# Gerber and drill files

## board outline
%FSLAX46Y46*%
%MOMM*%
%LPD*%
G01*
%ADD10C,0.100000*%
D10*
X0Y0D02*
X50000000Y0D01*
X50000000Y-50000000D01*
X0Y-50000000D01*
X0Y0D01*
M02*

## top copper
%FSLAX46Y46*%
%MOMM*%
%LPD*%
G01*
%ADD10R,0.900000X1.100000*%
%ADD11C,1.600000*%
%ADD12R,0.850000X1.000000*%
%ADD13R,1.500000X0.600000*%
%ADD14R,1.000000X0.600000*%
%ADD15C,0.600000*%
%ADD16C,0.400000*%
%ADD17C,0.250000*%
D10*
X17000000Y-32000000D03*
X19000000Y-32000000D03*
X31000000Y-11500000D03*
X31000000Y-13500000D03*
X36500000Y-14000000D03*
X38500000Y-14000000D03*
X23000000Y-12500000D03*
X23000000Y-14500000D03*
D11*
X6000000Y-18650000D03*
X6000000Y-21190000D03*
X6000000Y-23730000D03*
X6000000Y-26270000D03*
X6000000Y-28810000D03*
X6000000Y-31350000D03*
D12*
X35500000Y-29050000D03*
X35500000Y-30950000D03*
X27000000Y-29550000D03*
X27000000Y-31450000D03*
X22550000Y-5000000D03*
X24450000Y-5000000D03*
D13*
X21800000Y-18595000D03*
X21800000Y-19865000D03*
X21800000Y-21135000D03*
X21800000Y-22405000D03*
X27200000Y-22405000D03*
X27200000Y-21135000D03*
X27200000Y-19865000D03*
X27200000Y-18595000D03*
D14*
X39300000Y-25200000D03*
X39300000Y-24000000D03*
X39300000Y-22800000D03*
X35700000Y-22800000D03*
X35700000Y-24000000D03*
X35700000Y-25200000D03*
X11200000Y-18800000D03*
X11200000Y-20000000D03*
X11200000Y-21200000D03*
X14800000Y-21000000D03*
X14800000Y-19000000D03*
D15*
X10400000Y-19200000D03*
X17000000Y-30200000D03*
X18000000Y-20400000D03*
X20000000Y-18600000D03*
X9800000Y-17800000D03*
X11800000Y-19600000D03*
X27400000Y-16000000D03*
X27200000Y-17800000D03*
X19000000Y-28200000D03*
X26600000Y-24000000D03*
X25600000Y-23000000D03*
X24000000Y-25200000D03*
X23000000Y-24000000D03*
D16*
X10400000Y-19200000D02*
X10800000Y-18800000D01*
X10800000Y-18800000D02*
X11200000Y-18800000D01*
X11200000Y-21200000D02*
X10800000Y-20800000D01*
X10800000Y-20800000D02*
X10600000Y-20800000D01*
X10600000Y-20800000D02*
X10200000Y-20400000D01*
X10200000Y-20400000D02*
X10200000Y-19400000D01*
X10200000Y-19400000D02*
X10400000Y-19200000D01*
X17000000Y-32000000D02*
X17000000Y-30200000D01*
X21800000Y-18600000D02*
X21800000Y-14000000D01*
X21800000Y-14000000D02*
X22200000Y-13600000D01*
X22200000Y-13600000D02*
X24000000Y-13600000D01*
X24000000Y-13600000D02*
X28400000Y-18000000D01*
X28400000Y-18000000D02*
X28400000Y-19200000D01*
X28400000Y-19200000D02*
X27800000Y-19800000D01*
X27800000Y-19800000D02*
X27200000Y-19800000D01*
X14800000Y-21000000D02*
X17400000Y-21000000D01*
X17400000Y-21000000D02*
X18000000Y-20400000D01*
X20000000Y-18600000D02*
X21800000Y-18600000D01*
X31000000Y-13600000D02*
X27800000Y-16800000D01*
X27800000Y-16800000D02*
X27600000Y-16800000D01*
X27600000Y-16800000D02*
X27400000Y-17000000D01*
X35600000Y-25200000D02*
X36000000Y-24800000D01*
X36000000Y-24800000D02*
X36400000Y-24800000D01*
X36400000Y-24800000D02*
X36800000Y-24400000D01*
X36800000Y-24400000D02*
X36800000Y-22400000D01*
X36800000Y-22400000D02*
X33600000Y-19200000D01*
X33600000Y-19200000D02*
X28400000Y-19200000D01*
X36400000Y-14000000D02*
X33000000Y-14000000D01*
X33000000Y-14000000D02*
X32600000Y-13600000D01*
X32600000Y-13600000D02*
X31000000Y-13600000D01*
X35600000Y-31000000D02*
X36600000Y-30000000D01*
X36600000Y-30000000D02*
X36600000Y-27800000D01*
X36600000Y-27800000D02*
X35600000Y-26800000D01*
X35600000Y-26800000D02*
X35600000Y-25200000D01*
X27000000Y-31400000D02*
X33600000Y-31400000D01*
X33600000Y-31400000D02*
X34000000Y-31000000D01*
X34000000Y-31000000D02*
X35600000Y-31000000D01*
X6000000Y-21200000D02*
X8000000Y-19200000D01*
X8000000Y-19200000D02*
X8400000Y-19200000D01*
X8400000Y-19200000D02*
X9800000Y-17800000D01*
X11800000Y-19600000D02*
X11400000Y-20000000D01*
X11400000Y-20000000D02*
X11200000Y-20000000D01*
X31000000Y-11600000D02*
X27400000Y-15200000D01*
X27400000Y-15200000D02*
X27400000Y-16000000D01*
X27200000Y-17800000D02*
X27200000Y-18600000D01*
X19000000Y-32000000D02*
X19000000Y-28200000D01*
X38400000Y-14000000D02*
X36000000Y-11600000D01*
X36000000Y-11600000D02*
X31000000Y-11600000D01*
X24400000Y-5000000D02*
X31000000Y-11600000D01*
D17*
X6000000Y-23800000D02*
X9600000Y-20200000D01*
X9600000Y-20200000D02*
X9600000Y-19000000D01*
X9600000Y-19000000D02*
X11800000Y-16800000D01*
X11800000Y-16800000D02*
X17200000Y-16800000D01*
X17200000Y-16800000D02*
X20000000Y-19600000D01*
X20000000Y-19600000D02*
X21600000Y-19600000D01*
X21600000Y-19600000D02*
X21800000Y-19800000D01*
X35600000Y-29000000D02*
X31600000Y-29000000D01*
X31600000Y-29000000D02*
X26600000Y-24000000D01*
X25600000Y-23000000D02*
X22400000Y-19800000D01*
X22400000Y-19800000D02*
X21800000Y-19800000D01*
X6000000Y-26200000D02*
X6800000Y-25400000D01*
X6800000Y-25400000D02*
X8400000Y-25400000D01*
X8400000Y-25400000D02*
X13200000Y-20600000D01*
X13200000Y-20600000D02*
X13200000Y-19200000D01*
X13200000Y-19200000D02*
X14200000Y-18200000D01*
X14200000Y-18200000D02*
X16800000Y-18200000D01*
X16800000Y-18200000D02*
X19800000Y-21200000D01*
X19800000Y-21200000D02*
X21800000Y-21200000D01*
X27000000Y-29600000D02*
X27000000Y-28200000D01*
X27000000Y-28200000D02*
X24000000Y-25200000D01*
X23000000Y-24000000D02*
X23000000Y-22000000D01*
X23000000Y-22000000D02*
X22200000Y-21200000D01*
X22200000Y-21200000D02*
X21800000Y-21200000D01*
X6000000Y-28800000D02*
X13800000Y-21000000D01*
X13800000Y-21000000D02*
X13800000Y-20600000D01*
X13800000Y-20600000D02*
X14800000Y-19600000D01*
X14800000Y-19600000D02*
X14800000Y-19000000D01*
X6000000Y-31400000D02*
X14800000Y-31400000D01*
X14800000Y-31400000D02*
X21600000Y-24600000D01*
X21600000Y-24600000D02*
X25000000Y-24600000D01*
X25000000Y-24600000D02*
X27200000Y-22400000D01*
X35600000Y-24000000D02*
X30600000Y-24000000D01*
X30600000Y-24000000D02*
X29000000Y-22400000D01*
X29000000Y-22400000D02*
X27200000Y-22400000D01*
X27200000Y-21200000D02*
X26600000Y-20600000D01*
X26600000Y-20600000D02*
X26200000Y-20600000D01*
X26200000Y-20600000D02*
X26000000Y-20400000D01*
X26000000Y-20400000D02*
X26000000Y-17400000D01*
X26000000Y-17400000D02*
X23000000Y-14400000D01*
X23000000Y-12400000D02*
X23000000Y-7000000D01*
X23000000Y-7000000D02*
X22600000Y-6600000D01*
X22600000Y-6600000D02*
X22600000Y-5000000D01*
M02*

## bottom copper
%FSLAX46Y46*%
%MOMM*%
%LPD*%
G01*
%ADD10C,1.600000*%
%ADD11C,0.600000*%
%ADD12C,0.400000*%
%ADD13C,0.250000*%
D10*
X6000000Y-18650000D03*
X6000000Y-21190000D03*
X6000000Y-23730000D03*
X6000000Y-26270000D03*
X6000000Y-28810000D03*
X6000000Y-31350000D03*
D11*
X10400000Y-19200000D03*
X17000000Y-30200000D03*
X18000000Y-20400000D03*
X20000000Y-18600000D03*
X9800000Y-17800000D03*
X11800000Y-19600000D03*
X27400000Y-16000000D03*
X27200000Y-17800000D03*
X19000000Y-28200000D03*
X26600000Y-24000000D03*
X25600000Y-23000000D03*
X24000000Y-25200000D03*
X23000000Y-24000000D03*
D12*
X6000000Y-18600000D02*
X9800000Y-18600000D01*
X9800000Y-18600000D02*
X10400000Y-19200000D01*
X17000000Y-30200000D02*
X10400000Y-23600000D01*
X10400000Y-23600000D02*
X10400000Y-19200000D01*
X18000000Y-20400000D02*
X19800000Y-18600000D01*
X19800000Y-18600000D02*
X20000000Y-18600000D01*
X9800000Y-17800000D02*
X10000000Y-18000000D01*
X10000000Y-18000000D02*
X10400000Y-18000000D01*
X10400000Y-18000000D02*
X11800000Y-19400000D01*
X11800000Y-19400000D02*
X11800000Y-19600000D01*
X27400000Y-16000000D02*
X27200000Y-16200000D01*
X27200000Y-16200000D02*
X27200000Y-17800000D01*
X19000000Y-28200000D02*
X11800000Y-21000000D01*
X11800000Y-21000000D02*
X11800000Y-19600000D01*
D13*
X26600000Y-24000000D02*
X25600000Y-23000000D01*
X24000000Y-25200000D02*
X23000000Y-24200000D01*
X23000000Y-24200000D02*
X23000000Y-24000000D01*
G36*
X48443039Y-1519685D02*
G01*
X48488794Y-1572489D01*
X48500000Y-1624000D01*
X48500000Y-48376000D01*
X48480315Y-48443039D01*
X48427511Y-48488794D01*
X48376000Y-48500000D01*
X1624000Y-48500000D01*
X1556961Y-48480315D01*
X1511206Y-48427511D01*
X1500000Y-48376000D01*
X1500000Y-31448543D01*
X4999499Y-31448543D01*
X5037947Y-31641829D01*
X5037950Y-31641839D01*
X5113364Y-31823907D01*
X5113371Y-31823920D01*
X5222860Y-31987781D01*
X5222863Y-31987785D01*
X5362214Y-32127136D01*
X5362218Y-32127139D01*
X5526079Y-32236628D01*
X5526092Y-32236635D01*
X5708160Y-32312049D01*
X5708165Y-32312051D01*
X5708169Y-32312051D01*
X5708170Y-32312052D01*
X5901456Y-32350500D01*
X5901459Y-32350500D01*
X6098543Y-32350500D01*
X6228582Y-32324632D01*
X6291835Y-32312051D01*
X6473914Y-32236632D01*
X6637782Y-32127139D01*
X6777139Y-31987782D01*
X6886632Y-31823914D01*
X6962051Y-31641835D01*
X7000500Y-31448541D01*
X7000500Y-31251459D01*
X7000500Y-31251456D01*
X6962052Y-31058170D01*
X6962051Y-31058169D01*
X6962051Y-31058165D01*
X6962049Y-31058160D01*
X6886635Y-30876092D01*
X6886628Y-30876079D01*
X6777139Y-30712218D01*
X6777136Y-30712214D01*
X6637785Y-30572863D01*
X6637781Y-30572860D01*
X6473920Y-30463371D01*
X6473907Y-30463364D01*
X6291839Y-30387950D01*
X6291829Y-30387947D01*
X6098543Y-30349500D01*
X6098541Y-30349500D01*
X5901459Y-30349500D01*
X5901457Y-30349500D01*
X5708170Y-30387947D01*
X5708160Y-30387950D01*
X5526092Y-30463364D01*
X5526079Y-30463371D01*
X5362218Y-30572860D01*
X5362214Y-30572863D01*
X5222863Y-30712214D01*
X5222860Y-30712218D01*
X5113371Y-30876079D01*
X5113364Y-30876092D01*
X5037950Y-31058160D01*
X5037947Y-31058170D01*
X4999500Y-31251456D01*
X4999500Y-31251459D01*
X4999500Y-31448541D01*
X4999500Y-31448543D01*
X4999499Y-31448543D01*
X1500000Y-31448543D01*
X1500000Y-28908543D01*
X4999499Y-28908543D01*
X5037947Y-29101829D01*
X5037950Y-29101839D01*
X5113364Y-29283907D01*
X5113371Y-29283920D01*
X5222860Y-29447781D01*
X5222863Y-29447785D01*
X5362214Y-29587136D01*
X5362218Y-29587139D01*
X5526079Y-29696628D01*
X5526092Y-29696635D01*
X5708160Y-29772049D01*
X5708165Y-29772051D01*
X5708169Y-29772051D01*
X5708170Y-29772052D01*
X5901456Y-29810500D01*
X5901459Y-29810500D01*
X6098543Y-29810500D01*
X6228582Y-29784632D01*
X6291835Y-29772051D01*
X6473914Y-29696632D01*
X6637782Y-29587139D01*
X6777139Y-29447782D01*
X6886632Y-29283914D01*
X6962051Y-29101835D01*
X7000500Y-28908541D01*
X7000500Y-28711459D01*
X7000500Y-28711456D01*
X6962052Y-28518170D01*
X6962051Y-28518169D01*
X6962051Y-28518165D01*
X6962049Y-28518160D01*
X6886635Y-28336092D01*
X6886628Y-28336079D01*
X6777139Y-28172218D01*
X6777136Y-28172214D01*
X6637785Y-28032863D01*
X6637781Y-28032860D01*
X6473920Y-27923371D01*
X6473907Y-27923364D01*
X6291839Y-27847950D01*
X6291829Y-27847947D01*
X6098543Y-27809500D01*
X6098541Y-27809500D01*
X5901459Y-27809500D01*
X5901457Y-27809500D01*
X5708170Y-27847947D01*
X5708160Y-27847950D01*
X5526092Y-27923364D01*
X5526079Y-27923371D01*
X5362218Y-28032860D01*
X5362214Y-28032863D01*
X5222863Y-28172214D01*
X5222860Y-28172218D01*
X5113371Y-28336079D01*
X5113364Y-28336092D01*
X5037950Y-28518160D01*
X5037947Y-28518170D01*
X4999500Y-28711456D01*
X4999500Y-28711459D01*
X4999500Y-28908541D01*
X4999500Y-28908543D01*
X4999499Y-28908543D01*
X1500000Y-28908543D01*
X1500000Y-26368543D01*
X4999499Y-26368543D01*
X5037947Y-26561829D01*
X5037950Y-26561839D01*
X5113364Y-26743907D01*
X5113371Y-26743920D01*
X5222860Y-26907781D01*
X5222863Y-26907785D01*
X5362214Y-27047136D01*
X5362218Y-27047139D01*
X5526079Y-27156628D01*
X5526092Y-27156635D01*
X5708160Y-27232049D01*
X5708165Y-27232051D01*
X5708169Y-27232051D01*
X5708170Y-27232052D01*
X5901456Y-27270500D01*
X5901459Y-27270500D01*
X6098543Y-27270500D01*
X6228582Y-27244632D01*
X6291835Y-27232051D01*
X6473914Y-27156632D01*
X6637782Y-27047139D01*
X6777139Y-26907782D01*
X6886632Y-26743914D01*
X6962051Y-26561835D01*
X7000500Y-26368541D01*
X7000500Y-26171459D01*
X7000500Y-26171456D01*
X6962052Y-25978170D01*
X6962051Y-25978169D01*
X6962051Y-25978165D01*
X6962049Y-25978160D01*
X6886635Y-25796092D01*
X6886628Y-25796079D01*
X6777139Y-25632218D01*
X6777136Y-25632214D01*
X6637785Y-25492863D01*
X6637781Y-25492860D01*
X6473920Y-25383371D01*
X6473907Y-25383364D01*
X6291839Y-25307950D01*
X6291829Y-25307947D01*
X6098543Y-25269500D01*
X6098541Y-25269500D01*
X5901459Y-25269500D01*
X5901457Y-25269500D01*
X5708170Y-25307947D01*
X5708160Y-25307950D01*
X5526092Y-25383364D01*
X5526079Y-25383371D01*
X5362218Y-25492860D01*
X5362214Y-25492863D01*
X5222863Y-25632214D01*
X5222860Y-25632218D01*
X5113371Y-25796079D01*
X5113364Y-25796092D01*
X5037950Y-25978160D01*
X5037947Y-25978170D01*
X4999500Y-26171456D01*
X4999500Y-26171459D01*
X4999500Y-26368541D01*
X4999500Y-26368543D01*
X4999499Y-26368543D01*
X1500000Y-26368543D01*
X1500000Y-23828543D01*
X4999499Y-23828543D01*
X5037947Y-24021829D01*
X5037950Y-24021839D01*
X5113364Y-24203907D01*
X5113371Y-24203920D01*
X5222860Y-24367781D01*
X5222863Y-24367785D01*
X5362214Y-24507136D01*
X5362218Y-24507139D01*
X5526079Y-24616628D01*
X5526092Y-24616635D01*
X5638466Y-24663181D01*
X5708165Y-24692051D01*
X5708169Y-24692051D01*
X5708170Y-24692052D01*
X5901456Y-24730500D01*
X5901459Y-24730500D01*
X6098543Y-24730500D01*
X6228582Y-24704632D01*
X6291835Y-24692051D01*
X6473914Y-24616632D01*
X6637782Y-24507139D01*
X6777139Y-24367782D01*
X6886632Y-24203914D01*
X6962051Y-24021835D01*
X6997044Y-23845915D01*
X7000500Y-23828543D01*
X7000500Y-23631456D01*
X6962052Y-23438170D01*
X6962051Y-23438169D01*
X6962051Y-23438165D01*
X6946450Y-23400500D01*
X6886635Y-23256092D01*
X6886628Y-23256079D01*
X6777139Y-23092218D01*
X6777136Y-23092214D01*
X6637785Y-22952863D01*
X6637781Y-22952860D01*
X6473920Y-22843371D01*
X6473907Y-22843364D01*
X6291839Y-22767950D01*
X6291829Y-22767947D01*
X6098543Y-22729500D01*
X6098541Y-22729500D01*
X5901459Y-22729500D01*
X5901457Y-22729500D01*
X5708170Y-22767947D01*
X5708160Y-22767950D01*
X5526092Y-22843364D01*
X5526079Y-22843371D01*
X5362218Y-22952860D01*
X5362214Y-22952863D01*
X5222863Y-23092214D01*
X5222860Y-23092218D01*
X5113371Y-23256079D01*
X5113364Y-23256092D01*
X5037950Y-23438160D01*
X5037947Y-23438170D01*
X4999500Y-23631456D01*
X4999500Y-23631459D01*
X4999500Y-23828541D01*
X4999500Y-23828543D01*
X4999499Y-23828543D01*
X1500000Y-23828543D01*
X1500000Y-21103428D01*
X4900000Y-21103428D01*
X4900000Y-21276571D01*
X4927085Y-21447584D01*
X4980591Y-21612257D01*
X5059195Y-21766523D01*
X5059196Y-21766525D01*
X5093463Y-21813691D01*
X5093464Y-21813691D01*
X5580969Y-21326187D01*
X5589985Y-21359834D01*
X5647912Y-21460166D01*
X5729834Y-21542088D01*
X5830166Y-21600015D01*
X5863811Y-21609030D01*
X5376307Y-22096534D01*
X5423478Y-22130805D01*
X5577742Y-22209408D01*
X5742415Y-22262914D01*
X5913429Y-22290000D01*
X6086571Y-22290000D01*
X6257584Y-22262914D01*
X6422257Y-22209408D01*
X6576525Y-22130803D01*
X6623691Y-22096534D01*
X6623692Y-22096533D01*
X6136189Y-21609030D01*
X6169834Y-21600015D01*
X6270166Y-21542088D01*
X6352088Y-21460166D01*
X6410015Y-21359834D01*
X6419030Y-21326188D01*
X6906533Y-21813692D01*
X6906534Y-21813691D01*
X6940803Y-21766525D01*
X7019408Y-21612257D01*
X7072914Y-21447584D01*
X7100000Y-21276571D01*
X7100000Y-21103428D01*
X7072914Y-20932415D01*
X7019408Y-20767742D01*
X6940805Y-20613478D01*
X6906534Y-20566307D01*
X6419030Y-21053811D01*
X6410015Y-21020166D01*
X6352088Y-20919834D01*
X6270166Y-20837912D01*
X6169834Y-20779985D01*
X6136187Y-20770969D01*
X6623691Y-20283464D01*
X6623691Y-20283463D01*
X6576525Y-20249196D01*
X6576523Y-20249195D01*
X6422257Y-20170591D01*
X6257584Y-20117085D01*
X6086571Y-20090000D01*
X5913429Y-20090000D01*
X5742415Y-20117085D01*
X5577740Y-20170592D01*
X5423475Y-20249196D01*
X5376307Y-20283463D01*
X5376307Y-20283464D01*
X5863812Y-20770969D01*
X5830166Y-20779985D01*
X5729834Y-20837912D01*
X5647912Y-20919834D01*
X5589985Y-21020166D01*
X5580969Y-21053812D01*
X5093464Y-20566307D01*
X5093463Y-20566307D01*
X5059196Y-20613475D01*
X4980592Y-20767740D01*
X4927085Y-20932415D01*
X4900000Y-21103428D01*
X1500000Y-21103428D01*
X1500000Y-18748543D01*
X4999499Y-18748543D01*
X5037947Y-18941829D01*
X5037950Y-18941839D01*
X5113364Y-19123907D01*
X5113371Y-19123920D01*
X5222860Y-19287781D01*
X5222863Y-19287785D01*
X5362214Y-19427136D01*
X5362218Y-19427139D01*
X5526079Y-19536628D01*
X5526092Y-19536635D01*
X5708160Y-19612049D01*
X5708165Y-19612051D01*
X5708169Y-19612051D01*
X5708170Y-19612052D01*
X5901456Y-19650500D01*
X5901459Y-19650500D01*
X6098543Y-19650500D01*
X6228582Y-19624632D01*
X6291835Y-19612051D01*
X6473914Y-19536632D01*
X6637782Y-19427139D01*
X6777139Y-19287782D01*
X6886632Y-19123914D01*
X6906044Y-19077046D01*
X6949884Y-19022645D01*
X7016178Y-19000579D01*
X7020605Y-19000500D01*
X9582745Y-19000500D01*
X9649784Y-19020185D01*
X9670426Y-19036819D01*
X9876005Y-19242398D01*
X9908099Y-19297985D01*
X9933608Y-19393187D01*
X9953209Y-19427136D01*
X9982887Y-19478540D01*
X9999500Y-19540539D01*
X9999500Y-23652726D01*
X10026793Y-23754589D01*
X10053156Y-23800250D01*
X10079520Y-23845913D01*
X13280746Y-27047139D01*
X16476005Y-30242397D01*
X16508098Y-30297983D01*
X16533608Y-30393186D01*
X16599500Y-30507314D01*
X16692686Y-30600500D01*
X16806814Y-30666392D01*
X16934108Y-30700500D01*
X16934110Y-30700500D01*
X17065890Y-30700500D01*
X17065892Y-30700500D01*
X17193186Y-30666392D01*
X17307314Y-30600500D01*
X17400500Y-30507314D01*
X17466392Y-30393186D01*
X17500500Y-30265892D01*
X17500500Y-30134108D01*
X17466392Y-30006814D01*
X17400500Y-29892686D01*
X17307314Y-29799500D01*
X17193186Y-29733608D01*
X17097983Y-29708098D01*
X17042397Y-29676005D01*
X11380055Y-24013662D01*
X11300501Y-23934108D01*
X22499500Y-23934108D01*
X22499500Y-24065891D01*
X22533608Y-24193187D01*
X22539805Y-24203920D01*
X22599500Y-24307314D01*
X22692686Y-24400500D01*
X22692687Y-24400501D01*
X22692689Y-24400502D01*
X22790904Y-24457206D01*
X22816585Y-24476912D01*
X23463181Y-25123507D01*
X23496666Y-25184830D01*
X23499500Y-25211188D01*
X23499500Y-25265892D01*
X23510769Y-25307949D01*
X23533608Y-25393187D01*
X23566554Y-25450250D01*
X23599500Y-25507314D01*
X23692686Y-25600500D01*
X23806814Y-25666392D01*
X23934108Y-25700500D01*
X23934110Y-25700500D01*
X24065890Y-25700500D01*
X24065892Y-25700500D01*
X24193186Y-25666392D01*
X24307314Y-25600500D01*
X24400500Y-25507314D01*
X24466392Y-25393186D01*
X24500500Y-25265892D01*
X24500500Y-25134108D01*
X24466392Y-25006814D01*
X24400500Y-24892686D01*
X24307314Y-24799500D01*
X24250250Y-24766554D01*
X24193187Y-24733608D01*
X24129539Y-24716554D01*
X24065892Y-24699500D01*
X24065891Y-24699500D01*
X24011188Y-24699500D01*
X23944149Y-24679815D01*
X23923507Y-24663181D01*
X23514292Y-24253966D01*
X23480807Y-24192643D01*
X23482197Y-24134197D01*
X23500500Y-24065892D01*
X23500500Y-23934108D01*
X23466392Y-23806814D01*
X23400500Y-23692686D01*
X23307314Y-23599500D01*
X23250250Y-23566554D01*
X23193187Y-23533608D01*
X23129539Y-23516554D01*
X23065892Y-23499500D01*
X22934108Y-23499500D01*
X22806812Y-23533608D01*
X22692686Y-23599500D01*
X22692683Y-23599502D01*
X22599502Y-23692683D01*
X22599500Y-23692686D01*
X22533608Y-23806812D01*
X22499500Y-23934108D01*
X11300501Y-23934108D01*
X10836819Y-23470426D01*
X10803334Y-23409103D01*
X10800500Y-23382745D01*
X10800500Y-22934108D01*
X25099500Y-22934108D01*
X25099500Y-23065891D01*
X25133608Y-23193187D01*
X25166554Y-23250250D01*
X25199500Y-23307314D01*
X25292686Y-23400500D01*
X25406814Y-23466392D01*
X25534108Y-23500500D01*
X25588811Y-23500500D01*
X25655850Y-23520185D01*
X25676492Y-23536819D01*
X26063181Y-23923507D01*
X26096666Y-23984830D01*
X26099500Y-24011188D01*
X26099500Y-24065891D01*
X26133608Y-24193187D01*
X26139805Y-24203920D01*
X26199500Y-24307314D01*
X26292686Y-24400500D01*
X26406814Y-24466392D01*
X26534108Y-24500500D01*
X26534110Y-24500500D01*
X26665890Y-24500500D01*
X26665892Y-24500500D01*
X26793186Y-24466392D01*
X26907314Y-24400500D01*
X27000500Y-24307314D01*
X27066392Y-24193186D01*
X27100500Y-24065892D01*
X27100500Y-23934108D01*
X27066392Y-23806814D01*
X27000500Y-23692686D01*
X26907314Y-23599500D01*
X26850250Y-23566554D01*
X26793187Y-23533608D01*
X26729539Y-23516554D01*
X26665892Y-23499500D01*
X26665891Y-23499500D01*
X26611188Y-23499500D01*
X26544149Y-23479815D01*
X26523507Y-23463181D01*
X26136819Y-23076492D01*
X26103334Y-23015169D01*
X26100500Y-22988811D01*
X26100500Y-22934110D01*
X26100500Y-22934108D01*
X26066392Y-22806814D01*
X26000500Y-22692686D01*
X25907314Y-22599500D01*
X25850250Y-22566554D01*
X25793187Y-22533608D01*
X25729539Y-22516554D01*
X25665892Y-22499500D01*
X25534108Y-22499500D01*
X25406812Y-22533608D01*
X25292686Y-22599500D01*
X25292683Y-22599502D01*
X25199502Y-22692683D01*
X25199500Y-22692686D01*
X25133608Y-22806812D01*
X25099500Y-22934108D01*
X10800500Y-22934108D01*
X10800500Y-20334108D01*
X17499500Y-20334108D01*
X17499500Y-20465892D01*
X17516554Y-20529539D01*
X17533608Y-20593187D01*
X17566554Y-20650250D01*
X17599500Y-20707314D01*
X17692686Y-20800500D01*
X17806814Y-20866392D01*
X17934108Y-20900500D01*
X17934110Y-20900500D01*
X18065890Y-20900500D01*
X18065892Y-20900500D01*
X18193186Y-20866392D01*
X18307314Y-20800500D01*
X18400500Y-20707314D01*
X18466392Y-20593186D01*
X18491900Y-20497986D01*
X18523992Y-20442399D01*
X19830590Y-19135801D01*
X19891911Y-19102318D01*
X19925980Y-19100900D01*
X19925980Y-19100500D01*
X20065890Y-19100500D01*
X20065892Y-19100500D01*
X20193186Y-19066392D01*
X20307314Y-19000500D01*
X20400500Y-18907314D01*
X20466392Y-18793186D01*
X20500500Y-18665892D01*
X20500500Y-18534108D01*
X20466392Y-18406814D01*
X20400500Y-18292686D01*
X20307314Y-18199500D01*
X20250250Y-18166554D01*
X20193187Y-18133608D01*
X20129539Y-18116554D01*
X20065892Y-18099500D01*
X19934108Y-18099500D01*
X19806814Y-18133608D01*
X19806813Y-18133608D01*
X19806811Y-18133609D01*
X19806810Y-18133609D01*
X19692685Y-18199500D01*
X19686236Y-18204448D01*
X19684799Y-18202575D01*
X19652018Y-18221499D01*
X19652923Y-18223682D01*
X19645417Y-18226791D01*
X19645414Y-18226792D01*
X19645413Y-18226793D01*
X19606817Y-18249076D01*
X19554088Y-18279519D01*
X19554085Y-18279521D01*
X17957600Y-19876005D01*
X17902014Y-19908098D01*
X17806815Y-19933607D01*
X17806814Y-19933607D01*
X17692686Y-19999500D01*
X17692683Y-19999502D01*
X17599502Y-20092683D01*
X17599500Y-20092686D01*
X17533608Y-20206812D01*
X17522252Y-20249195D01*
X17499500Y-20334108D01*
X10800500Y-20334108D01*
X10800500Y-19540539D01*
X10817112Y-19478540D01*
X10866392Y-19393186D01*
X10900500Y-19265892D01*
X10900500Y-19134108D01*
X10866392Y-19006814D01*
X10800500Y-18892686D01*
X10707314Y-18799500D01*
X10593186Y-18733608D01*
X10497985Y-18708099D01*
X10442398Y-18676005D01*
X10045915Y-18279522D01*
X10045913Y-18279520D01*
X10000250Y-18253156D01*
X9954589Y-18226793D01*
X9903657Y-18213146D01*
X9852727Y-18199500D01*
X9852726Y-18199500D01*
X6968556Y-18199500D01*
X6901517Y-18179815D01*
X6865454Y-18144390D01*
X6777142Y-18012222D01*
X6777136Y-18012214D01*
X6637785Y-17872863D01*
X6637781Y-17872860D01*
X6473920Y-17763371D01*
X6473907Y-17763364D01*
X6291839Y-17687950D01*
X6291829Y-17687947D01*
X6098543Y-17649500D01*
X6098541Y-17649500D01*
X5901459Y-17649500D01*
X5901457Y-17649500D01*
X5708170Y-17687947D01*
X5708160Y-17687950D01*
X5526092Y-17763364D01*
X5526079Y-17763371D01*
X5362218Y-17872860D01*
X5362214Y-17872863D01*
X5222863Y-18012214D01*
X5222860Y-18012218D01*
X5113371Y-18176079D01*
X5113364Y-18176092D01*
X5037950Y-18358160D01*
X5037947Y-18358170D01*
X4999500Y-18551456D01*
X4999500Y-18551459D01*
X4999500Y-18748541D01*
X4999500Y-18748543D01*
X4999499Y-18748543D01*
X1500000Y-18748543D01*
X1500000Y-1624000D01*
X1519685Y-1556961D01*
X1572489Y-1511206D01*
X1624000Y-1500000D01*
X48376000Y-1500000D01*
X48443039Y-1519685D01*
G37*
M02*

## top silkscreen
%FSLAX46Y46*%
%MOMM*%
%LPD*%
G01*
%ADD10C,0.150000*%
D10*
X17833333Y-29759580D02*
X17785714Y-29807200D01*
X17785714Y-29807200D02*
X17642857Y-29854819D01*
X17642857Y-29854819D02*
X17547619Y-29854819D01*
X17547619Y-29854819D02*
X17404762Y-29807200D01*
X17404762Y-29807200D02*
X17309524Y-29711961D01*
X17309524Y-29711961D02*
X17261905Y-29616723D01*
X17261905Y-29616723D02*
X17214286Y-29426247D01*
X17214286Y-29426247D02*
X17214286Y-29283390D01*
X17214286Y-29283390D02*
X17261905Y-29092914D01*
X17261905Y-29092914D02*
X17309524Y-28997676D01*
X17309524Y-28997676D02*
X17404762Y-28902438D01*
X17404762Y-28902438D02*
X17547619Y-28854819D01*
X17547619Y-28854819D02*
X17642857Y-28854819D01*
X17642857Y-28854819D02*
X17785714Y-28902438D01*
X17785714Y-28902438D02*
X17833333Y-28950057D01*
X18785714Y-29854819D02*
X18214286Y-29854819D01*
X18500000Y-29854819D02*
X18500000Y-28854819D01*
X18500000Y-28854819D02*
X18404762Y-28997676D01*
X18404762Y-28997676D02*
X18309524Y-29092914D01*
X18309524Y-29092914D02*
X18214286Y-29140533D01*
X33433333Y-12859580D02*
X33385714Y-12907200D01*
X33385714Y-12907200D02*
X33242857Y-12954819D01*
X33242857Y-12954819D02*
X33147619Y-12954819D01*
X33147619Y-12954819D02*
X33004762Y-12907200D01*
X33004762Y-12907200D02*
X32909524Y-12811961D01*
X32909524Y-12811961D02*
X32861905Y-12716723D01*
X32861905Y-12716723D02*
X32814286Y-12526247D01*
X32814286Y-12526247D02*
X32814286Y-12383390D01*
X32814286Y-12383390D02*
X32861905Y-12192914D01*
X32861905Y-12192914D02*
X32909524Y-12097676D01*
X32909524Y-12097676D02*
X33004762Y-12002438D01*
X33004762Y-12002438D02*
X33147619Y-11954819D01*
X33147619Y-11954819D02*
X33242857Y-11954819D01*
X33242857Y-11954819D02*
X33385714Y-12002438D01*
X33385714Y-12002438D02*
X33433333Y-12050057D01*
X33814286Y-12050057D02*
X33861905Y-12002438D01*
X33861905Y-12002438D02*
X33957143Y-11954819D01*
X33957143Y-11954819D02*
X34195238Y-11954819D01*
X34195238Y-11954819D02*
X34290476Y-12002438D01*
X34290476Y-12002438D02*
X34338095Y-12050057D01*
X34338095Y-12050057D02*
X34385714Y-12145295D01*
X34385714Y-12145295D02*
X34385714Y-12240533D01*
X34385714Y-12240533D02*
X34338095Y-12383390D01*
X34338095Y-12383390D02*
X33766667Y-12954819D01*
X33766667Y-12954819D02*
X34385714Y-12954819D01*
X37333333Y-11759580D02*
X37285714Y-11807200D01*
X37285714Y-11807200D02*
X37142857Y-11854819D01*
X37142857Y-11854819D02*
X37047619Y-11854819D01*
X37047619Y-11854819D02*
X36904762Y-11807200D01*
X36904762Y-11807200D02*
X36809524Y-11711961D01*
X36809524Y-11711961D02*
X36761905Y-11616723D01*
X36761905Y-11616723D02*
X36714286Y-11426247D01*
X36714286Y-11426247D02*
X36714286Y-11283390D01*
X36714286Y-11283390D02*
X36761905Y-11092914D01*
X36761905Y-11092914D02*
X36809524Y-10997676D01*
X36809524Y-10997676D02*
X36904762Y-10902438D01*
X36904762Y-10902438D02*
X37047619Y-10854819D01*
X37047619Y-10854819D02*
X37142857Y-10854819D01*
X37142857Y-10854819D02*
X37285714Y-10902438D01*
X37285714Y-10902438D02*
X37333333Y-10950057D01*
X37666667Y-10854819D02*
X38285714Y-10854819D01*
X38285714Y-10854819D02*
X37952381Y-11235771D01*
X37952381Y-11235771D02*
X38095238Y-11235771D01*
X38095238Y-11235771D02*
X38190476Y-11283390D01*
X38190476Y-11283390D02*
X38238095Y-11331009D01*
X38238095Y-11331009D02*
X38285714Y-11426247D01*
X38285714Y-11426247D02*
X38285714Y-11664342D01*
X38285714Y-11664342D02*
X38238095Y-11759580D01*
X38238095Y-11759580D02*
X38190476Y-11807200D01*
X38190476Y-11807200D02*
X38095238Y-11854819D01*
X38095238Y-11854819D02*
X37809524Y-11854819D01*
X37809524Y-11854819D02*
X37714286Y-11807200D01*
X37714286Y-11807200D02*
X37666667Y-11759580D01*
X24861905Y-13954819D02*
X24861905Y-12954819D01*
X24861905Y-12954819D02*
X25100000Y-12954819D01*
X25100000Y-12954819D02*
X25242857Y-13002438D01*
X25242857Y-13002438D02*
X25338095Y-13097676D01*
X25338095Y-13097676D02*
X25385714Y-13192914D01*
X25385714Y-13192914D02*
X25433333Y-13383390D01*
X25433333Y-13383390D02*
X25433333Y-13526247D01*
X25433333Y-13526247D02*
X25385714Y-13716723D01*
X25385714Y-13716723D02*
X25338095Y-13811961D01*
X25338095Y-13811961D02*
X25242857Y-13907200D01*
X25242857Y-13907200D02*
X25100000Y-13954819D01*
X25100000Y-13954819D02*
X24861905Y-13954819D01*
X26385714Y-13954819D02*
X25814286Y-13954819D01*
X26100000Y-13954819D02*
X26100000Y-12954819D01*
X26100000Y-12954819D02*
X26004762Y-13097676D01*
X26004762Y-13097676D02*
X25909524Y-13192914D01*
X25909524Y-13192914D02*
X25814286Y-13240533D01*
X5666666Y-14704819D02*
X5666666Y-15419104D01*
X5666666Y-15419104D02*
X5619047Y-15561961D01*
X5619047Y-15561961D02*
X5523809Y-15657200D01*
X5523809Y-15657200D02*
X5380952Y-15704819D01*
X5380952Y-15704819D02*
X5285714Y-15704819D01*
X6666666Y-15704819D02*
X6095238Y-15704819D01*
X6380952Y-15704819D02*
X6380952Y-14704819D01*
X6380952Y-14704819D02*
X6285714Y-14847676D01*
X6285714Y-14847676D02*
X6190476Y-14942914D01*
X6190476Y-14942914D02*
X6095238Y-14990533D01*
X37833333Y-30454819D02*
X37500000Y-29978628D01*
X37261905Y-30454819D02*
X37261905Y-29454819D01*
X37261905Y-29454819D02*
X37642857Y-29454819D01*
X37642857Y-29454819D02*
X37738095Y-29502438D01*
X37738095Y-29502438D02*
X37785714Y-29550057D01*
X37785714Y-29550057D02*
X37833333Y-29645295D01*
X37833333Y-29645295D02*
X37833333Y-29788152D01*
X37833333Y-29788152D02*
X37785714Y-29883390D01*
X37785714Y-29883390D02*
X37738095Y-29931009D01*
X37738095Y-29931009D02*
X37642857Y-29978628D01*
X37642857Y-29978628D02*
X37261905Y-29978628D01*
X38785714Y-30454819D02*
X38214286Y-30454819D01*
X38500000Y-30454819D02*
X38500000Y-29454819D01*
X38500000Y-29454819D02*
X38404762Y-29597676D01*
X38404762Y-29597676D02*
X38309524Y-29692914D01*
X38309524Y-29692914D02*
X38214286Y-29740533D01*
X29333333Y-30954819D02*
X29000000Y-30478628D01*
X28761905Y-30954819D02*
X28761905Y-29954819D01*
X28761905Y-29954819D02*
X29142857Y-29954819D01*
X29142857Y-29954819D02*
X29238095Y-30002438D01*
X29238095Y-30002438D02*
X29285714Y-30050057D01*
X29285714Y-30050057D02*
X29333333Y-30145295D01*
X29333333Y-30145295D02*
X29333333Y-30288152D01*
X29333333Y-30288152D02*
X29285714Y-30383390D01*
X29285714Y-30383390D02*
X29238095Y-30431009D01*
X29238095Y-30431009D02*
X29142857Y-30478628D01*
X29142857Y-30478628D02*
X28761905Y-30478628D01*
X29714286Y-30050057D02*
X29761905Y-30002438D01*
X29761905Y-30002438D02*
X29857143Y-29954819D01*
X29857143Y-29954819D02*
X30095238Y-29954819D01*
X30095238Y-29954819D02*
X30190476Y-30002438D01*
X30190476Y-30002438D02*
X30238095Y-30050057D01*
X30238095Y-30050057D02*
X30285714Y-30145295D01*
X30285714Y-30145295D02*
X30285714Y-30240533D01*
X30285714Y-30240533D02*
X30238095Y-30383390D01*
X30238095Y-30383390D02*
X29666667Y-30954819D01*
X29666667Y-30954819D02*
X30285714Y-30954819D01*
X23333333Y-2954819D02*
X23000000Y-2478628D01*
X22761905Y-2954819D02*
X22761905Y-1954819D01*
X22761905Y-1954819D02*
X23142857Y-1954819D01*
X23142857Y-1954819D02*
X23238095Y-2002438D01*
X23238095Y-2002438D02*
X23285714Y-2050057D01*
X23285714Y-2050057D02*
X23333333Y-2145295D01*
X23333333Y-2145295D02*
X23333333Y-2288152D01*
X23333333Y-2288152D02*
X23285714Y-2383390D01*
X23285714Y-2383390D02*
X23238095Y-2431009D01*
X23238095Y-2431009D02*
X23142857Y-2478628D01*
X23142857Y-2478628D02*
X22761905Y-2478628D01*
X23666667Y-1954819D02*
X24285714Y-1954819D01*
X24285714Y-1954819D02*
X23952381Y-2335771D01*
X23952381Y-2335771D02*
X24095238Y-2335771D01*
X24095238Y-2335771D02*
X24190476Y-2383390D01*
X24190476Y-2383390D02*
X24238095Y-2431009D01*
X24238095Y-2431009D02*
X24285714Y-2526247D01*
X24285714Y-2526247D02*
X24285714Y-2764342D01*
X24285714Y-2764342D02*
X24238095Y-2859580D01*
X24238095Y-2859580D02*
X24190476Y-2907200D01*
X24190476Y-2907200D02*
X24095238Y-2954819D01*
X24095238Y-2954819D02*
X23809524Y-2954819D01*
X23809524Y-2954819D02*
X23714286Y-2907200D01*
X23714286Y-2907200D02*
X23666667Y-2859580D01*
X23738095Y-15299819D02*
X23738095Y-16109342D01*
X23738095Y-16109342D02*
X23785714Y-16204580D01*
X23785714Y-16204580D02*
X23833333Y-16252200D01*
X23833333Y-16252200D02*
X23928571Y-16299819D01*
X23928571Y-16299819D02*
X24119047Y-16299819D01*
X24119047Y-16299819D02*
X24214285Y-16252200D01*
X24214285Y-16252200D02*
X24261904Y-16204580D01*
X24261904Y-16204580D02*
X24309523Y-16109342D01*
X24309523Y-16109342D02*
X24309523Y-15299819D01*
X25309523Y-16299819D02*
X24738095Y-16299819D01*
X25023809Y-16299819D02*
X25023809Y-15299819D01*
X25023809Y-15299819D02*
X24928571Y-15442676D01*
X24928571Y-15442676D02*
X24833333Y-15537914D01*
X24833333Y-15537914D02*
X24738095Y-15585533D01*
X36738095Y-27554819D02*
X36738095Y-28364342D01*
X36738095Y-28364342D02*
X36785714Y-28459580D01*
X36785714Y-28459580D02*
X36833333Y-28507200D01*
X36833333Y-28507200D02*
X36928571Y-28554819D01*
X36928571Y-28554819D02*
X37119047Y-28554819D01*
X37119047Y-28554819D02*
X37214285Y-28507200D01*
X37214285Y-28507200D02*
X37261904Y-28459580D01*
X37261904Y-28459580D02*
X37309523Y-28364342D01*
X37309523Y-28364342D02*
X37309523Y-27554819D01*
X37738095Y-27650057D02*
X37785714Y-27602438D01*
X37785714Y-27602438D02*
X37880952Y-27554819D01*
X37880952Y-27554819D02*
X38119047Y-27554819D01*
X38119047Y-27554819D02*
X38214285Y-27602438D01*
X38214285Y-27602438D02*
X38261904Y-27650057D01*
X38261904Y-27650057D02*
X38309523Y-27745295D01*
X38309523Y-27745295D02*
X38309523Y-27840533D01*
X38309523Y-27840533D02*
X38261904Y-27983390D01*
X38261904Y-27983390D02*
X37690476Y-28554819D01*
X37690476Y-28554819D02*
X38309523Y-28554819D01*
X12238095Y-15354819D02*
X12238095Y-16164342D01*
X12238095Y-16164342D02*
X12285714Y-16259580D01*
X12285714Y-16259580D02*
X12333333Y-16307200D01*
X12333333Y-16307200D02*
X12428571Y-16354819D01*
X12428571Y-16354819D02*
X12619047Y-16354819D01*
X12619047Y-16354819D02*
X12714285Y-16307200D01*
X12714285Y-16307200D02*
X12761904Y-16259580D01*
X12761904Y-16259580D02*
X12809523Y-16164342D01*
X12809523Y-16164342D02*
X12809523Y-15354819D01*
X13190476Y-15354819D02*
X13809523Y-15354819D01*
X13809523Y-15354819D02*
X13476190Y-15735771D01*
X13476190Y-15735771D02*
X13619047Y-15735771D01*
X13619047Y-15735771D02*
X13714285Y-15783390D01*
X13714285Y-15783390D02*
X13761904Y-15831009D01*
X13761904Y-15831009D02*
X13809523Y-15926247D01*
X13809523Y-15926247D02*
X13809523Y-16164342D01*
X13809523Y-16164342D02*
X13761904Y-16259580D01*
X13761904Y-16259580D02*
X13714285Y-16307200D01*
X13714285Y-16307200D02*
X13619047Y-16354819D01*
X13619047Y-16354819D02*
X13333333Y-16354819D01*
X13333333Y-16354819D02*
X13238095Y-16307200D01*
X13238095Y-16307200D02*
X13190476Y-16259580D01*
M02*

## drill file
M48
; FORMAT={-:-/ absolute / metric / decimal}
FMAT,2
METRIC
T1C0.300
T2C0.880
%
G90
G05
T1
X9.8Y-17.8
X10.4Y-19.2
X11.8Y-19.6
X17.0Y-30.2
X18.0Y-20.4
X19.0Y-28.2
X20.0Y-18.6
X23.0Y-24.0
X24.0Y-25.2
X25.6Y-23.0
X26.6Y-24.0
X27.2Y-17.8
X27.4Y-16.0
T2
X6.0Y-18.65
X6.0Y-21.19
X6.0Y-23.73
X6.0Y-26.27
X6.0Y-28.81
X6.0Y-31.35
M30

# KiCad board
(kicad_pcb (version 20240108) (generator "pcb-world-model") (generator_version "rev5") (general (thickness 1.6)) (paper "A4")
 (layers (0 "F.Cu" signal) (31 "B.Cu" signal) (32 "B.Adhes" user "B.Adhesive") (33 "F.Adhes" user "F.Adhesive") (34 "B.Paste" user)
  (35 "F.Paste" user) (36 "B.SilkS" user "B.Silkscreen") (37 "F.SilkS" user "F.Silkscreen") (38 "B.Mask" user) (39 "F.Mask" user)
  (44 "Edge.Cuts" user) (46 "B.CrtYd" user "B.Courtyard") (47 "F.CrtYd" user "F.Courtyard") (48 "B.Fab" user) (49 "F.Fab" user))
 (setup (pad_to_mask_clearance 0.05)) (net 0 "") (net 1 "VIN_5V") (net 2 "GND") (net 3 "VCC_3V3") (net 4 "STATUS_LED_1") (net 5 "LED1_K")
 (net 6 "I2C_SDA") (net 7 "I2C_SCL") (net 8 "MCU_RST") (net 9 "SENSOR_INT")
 (gr_rect (start 0.0 0.0) (end 50.0000 50.0000) (stroke (width 0.1) (type default)) (fill none) (layer "Edge.Cuts"))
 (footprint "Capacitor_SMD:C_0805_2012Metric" (layer "F.Cu") (at 18.0000 32.0000 0)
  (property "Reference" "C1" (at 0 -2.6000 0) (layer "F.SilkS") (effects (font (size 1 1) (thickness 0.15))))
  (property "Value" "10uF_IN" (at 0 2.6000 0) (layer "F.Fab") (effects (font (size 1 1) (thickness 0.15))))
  (pad "1" smd rect (at -1.0000 0.0000) (size 0.9000 1.1000) (layers "F.Cu" "F.Paste" "F.Mask") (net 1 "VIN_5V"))
  (pad "2" smd rect (at 1.0000 0.0000) (size 0.9000 1.1000) (layers "F.Cu" "F.Paste" "F.Mask") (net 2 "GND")))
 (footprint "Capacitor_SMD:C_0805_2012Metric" (layer "F.Cu") (at 31.0000 12.5000 270)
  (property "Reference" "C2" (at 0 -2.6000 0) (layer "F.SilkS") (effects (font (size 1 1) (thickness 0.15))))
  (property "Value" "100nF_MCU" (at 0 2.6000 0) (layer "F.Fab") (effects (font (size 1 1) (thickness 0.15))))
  (pad "1" smd rect (at -1.0000 0.0000) (size 0.9000 1.1000) (layers "F.Cu" "F.Paste" "F.Mask") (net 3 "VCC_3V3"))
  (pad "2" smd rect (at 1.0000 0.0000) (size 0.9000 1.1000) (layers "F.Cu" "F.Paste" "F.Mask") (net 2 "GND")))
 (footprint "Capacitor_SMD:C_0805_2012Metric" (layer "F.Cu") (at 37.5000 14.0000 0)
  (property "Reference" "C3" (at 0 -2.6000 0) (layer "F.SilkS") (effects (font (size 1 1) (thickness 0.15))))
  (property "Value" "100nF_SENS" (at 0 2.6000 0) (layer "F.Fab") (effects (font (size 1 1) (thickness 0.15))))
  (pad "1" smd rect (at -1.0000 0.0000) (size 0.9000 1.1000) (layers "F.Cu" "F.Paste" "F.Mask") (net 3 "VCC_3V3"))
  (pad "2" smd rect (at 1.0000 0.0000) (size 0.9000 1.1000) (layers "F.Cu" "F.Paste" "F.Mask") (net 2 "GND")))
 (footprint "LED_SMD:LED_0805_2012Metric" (layer "F.Cu") (at 23.0000 13.5000 270)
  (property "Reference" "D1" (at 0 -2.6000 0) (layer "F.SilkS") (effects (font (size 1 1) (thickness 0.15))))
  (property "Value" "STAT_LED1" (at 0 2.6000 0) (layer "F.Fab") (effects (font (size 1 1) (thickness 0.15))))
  (pad "1" smd rect (at -1.0000 0.0000) (size 0.9000 1.1000) (layers "F.Cu" "F.Paste" "F.Mask") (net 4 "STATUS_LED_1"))
  (pad "2" smd rect (at 1.0000 0.0000) (size 0.9000 1.1000) (layers "F.Cu" "F.Paste" "F.Mask") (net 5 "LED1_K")))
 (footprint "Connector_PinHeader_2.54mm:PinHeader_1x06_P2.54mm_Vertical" (layer "F.Cu") (at 6.0000 25.0000 0) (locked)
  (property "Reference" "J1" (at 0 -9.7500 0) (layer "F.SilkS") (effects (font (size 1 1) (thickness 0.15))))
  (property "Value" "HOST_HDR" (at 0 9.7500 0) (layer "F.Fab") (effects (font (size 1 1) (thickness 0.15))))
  (pad "1" thru_hole circle (at 0.0000 -6.3500) (size 1.6000 1.6000) (drill 0.8800) (layers "*.Cu" "*.Mask") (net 1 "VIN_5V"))
  (pad "2" thru_hole circle (at 0.0000 -3.8100) (size 1.6000 1.6000) (drill 0.8800) (layers "*.Cu" "*.Mask") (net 2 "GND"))
  (pad "3" thru_hole circle (at 0.0000 -1.2700) (size 1.6000 1.6000) (drill 0.8800) (layers "*.Cu" "*.Mask") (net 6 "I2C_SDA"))
  (pad "4" thru_hole circle (at 0.0000 1.2700) (size 1.6000 1.6000) (drill 0.8800) (layers "*.Cu" "*.Mask") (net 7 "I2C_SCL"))
  (pad "5" thru_hole circle (at 0.0000 3.8100) (size 1.6000 1.6000) (drill 0.8800) (layers "*.Cu" "*.Mask") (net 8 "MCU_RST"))
  (pad "6" thru_hole circle (at 0.0000 6.3500) (size 1.6000 1.6000) (drill 0.8800) (layers "*.Cu" "*.Mask") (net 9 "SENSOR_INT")))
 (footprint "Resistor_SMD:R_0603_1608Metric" (layer "F.Cu") (at 35.5000 30.0000 270)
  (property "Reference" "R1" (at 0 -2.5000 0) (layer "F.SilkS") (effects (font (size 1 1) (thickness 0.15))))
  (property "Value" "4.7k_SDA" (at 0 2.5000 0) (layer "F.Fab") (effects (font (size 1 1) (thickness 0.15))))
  (pad "1" smd rect (at -0.9500 0.0000) (size 0.8500 1.0000) (layers "F.Cu" "F.Paste" "F.Mask") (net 3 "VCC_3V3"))
  (pad "2" smd rect (at 0.9500 0.0000) (size 0.8500 1.0000) (layers "F.Cu" "F.Paste" "F.Mask") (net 6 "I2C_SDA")))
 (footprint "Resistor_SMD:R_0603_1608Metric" (layer "F.Cu") (at 27.0000 30.5000 270)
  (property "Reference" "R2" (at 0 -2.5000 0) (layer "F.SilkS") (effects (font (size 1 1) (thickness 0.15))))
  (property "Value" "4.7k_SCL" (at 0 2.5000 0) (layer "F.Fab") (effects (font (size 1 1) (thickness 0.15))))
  (pad "1" smd rect (at -0.9500 0.0000) (size 0.8500 1.0000) (layers "F.Cu" "F.Paste" "F.Mask") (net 3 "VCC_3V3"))
  (pad "2" smd rect (at 0.9500 0.0000) (size 0.8500 1.0000) (layers "F.Cu" "F.Paste" "F.Mask") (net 7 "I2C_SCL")))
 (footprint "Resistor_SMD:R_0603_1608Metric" (layer "F.Cu") (at 23.5000 5.0000 0)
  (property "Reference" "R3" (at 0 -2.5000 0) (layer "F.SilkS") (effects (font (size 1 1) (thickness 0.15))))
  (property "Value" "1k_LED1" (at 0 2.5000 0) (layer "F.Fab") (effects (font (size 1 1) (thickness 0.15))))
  (pad "1" smd rect (at -0.9500 0.0000) (size 0.8500 1.0000) (layers "F.Cu" "F.Paste" "F.Mask") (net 5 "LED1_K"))
  (pad "2" smd rect (at 0.9500 0.0000) (size 0.8500 1.0000) (layers "F.Cu" "F.Paste" "F.Mask") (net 2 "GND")))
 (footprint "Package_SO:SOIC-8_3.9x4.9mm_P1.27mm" (layer "F.Cu") (at 24.5000 20.5000 0)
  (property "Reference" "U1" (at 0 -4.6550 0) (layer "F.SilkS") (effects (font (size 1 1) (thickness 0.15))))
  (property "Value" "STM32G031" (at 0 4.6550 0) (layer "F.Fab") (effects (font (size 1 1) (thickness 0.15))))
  (pad "1" smd rect (at -2.7000 -1.9050) (size 1.5000 0.6000) (layers "F.Cu" "F.Paste" "F.Mask") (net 3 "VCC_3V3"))
  (pad "2" smd rect (at -2.7000 -0.6350) (size 1.5000 0.6000) (layers "F.Cu" "F.Paste" "F.Mask") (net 6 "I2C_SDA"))
  (pad "3" smd rect (at -2.7000 0.6350) (size 1.5000 0.6000) (layers "F.Cu" "F.Paste" "F.Mask") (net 7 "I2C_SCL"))
  (pad "4" smd rect (at -2.7000 1.9050) (size 1.5000 0.6000) (layers "F.Cu" "F.Paste" "F.Mask") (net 8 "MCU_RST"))
  (pad "5" smd rect (at 2.7000 1.9050) (size 1.5000 0.6000) (layers "F.Cu" "F.Paste" "F.Mask") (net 9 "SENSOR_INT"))
  (pad "6" smd rect (at 2.7000 0.6350) (size 1.5000 0.6000) (layers "F.Cu" "F.Paste" "F.Mask") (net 4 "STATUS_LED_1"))
  (pad "7" smd rect (at 2.7000 -0.6350) (size 1.5000 0.6000) (layers "F.Cu" "F.Paste" "F.Mask") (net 3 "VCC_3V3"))
  (pad "8" smd rect (at 2.7000 -1.9050) (size 1.5000 0.6000) (layers "F.Cu" "F.Paste" "F.Mask") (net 2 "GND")))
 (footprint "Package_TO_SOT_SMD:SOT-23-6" (layer "F.Cu") (at 37.5000 24.0000 180)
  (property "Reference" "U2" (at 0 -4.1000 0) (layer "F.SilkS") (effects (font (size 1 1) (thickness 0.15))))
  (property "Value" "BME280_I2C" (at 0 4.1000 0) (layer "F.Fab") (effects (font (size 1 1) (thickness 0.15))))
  (pad "1" smd rect (at -1.8000 -1.2000) (size 1.0000 0.6000) (layers "F.Cu" "F.Paste" "F.Mask") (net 3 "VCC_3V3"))
  (pad "2" smd rect (at -1.8000 0.0000) (size 1.0000 0.6000) (layers "F.Cu" "F.Paste" "F.Mask") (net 2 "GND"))
  (pad "3" smd rect (at -1.8000 1.2000) (size 1.0000 0.6000) (layers "F.Cu" "F.Paste" "F.Mask") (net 6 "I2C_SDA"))
  (pad "4" smd rect (at 1.8000 1.2000) (size 1.0000 0.6000) (layers "F.Cu" "F.Paste" "F.Mask") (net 7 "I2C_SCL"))
  (pad "5" smd rect (at 1.8000 0.0000) (size 1.0000 0.6000) (layers "F.Cu" "F.Paste" "F.Mask") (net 9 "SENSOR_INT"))
  (pad "6" smd rect (at 1.8000 -1.2000) (size 1.0000 0.6000) (layers "F.Cu" "F.Paste" "F.Mask") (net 3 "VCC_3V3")))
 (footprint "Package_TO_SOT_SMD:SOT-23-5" (layer "F.Cu") (at 13.0000 20.0000 0)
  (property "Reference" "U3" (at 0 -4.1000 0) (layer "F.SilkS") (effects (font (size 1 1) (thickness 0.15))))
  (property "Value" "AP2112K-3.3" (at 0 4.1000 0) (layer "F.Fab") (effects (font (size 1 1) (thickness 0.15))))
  (pad "1" smd rect (at -1.8000 -1.2000) (size 1.0000 0.6000) (layers "F.Cu" "F.Paste" "F.Mask") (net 1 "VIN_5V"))
  (pad "2" smd rect (at -1.8000 0.0000) (size 1.0000 0.6000) (layers "F.Cu" "F.Paste" "F.Mask") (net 2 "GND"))
  (pad "3" smd rect (at -1.8000 1.2000) (size 1.0000 0.6000) (layers "F.Cu" "F.Paste" "F.Mask") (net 1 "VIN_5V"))
  (pad "4" smd rect (at 1.8000 1.0000) (size 1.0000 0.6000) (layers "F.Cu" "F.Paste" "F.Mask") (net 3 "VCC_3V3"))
  (pad "5" smd rect (at 1.8000 -1.0000) (size 1.0000 0.6000) (layers "F.Cu" "F.Paste" "F.Mask") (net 8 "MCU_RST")))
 (segment (start 6.0000 18.6000) (end 9.8000 18.6000) (width 0.4000) (layer "B.Cu") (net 1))
 (segment (start 9.8000 18.6000) (end 10.4000 19.2000) (width 0.4000) (layer "B.Cu") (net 1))
 (segment (start 10.4000 19.2000) (end 10.8000 18.8000) (width 0.4000) (layer "F.Cu") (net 1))
 (segment (start 10.8000 18.8000) (end 11.2000 18.8000) (width 0.4000) (layer "F.Cu") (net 1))
 (segment (start 11.2000 21.2000) (end 10.8000 20.8000) (width 0.4000) (layer "F.Cu") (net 1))
 (segment (start 10.8000 20.8000) (end 10.6000 20.8000) (width 0.4000) (layer "F.Cu") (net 1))
 (segment (start 10.6000 20.8000) (end 10.2000 20.4000) (width 0.4000) (layer "F.Cu") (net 1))
 (segment (start 10.2000 20.4000) (end 10.2000 19.4000) (width 0.4000) (layer "F.Cu") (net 1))
 (segment (start 10.2000 19.4000) (end 10.4000 19.2000) (width 0.4000) (layer "F.Cu") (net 1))
 (segment (start 17.0000 32.0000) (end 17.0000 30.2000) (width 0.4000) (layer "F.Cu") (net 1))
 (segment (start 17.0000 30.2000) (end 10.4000 23.6000) (width 0.4000) (layer "B.Cu") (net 1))
 (segment (start 10.4000 23.6000) (end 10.4000 19.2000) (width 0.4000) (layer "B.Cu") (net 1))
 (segment (start 21.8000 18.6000) (end 21.8000 14.0000) (width 0.4000) (layer "F.Cu") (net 3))
 (segment (start 21.8000 14.0000) (end 22.2000 13.6000) (width 0.4000) (layer "F.Cu") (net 3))
 (segment (start 22.2000 13.6000) (end 24.0000 13.6000) (width 0.4000) (layer "F.Cu") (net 3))
 (segment (start 24.0000 13.6000) (end 28.4000 18.0000) (width 0.4000) (layer "F.Cu") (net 3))
 (segment (start 28.4000 18.0000) (end 28.4000 19.2000) (width 0.4000) (layer "F.Cu") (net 3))
 (segment (start 28.4000 19.2000) (end 27.8000 19.8000) (width 0.4000) (layer "F.Cu") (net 3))
 (segment (start 27.8000 19.8000) (end 27.2000 19.8000) (width 0.4000) (layer "F.Cu") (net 3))
 (segment (start 14.8000 21.0000) (end 17.4000 21.0000) (width 0.4000) (layer "F.Cu") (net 3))
 (segment (start 17.4000 21.0000) (end 18.0000 20.4000) (width 0.4000) (layer "F.Cu") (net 3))
 (segment (start 18.0000 20.4000) (end 19.8000 18.6000) (width 0.4000) (layer "B.Cu") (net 3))
 (segment (start 19.8000 18.6000) (end 20.0000 18.6000) (width 0.4000) (layer "B.Cu") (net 3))
 (segment (start 20.0000 18.6000) (end 21.8000 18.6000) (width 0.4000) (layer "F.Cu") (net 3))
 (segment (start 31.0000 13.6000) (end 27.8000 16.8000) (width 0.4000) (layer "F.Cu") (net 3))
 (segment (start 27.8000 16.8000) (end 27.6000 16.8000) (width 0.4000) (layer "F.Cu") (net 3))
 (segment (start 27.6000 16.8000) (end 27.4000 17.0000) (width 0.4000) (layer "F.Cu") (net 3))
 (segment (start 35.6000 25.2000) (end 36.0000 24.8000) (width 0.4000) (layer "F.Cu") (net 3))
 (segment (start 36.0000 24.8000) (end 36.4000 24.8000) (width 0.4000) (layer "F.Cu") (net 3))
 (segment (start 36.4000 24.8000) (end 36.8000 24.4000) (width 0.4000) (layer "F.Cu") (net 3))
 (segment (start 36.8000 24.4000) (end 36.8000 22.4000) (width 0.4000) (layer "F.Cu") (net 3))
 (segment (start 36.8000 22.4000) (end 33.6000 19.2000) (width 0.4000) (layer "F.Cu") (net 3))
 (segment (start 33.6000 19.2000) (end 28.4000 19.2000) (width 0.4000) (layer "F.Cu") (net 3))
 (segment (start 36.4000 14.0000) (end 33.0000 14.0000) (width 0.4000) (layer "F.Cu") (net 3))
 (segment (start 33.0000 14.0000) (end 32.6000 13.6000) (width 0.4000) (layer "F.Cu") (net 3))
 (segment (start 32.6000 13.6000) (end 31.0000 13.6000) (width 0.4000) (layer "F.Cu") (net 3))
 (segment (start 35.6000 31.0000) (end 36.6000 30.0000) (width 0.4000) (layer "F.Cu") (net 3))
 (segment (start 36.6000 30.0000) (end 36.6000 27.8000) (width 0.4000) (layer "F.Cu") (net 3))
 (segment (start 36.6000 27.8000) (end 35.6000 26.8000) (width 0.4000) (layer "F.Cu") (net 3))
 (segment (start 35.6000 26.8000) (end 35.6000 25.2000) (width 0.4000) (layer "F.Cu") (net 3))
 (segment (start 27.0000 31.4000) (end 33.6000 31.4000) (width 0.4000) (layer "F.Cu") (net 3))
 (segment (start 33.6000 31.4000) (end 34.0000 31.0000) (width 0.4000) (layer "F.Cu") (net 3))
 (segment (start 34.0000 31.0000) (end 35.6000 31.0000) (width 0.4000) (layer "F.Cu") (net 3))
 (segment (start 6.0000 21.2000) (end 8.0000 19.2000) (width 0.4000) (layer "F.Cu") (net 2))
 (segment (start 8.0000 19.2000) (end 8.4000 19.2000) (width 0.4000) (layer "F.Cu") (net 2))
 (segment (start 8.4000 19.2000) (end 9.8000 17.8000) (width 0.4000) (layer "F.Cu") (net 2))
 (segment (start 9.8000 17.8000) (end 10.0000 18.0000) (width 0.4000) (layer "B.Cu") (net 2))
 (segment (start 10.0000 18.0000) (end 10.4000 18.0000) (width 0.4000) (layer "B.Cu") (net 2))
 (segment (start 10.4000 18.0000) (end 11.8000 19.4000) (width 0.4000) (layer "B.Cu") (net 2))
 (segment (start 11.8000 19.4000) (end 11.8000 19.6000) (width 0.4000) (layer "B.Cu") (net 2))
 (segment (start 11.8000 19.6000) (end 11.4000 20.0000) (width 0.4000) (layer "F.Cu") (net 2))
 (segment (start 11.4000 20.0000) (end 11.2000 20.0000) (width 0.4000) (layer "F.Cu") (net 2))
 (segment (start 31.0000 11.6000) (end 27.4000 15.2000) (width 0.4000) (layer "F.Cu") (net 2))
 (segment (start 27.4000 15.2000) (end 27.4000 16.0000) (width 0.4000) (layer "F.Cu") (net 2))
 (segment (start 27.4000 16.0000) (end 27.2000 16.2000) (width 0.4000) (layer "B.Cu") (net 2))
 (segment (start 27.2000 16.2000) (end 27.2000 17.8000) (width 0.4000) (layer "B.Cu") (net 2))
 (segment (start 27.2000 17.8000) (end 27.2000 18.6000) (width 0.4000) (layer "F.Cu") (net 2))
 (segment (start 19.0000 32.0000) (end 19.0000 28.2000) (width 0.4000) (layer "F.Cu") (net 2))
 (segment (start 19.0000 28.2000) (end 11.8000 21.0000) (width 0.4000) (layer "B.Cu") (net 2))
 (segment (start 11.8000 21.0000) (end 11.8000 19.6000) (width 0.4000) (layer "B.Cu") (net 2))
 (segment (start 38.4000 14.0000) (end 36.0000 11.6000) (width 0.4000) (layer "F.Cu") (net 2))
 (segment (start 36.0000 11.6000) (end 31.0000 11.6000) (width 0.4000) (layer "F.Cu") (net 2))
 (segment (start 24.4000 5.0000) (end 31.0000 11.6000) (width 0.4000) (layer "F.Cu") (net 2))
 (segment (start 6.0000 23.8000) (end 9.6000 20.2000) (width 0.2500) (layer "F.Cu") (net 6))
 (segment (start 9.6000 20.2000) (end 9.6000 19.0000) (width 0.2500) (layer "F.Cu") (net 6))
 (segment (start 9.6000 19.0000) (end 11.8000 16.8000) (width 0.2500) (layer "F.Cu") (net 6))
 (segment (start 11.8000 16.8000) (end 17.2000 16.8000) (width 0.2500) (layer "F.Cu") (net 6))
 (segment (start 17.2000 16.8000) (end 20.0000 19.6000) (width 0.2500) (layer "F.Cu") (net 6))
 (segment (start 20.0000 19.6000) (end 21.6000 19.6000) (width 0.2500) (layer "F.Cu") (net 6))
 (segment (start 21.6000 19.6000) (end 21.8000 19.8000) (width 0.2500) (layer "F.Cu") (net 6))
 (segment (start 35.6000 29.0000) (end 31.6000 29.0000) (width 0.2500) (layer "F.Cu") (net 6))
 (segment (start 31.6000 29.0000) (end 26.6000 24.0000) (width 0.2500) (layer "F.Cu") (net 6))
 (segment (start 26.6000 24.0000) (end 25.6000 23.0000) (width 0.2500) (layer "B.Cu") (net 6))
 (segment (start 25.6000 23.0000) (end 22.4000 19.8000) (width 0.2500) (layer "F.Cu") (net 6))
 (segment (start 22.4000 19.8000) (end 21.8000 19.8000) (width 0.2500) (layer "F.Cu") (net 6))
 (segment (start 6.0000 26.2000) (end 6.8000 25.4000) (width 0.2500) (layer "F.Cu") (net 7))
 (segment (start 6.8000 25.4000) (end 8.4000 25.4000) (width 0.2500) (layer "F.Cu") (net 7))
 (segment (start 8.4000 25.4000) (end 13.2000 20.6000) (width 0.2500) (layer "F.Cu") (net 7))
 (segment (start 13.2000 20.6000) (end 13.2000 19.2000) (width 0.2500) (layer "F.Cu") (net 7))
 (segment (start 13.2000 19.2000) (end 14.2000 18.2000) (width 0.2500) (layer "F.Cu") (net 7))
 (segment (start 14.2000 18.2000) (end 16.8000 18.2000) (width 0.2500) (layer "F.Cu") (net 7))
 (segment (start 16.8000 18.2000) (end 19.8000 21.2000) (width 0.2500) (layer "F.Cu") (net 7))
 (segment (start 19.8000 21.2000) (end 21.8000 21.2000) (width 0.2500) (layer "F.Cu") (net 7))
 (segment (start 27.0000 29.6000) (end 27.0000 28.2000) (width 0.2500) (layer "F.Cu") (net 7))
 (segment (start 27.0000 28.2000) (end 24.0000 25.2000) (width 0.2500) (layer "F.Cu") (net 7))
 (segment (start 24.0000 25.2000) (end 23.0000 24.2000) (width 0.2500) (layer "B.Cu") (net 7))
 (segment (start 23.0000 24.2000) (end 23.0000 24.0000) (width 0.2500) (layer "B.Cu") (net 7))
 (segment (start 23.0000 24.0000) (end 23.0000 22.0000) (width 0.2500) (layer "F.Cu") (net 7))
 (segment (start 23.0000 22.0000) (end 22.2000 21.2000) (width 0.2500) (layer "F.Cu") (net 7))
 (segment (start 22.2000 21.2000) (end 21.8000 21.2000) (width 0.2500) (layer "F.Cu") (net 7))
 (segment (start 6.0000 28.8000) (end 13.8000 21.0000) (width 0.2500) (layer "F.Cu") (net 8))
 (segment (start 13.8000 21.0000) (end 13.8000 20.6000) (width 0.2500) (layer "F.Cu") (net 8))
 (segment (start 13.8000 20.6000) (end 14.8000 19.6000) (width 0.2500) (layer "F.Cu") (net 8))
 (segment (start 14.8000 19.6000) (end 14.8000 19.0000) (width 0.2500) (layer "F.Cu") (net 8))
 (segment (start 6.0000 31.4000) (end 14.8000 31.4000) (width 0.2500) (layer "F.Cu") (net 9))
 (segment (start 14.8000 31.4000) (end 21.6000 24.6000) (width 0.2500) (layer "F.Cu") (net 9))
 (segment (start 21.6000 24.6000) (end 25.0000 24.6000) (width 0.2500) (layer "F.Cu") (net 9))
 (segment (start 25.0000 24.6000) (end 27.2000 22.4000) (width 0.2500) (layer "F.Cu") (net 9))
 (segment (start 35.6000 24.0000) (end 30.6000 24.0000) (width 0.2500) (layer "F.Cu") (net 9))
 (segment (start 30.6000 24.0000) (end 29.0000 22.4000) (width 0.2500) (layer "F.Cu") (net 9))
 (segment (start 29.0000 22.4000) (end 27.2000 22.4000) (width 0.2500) (layer "F.Cu") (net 9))
 (segment (start 27.2000 21.2000) (end 26.6000 20.6000) (width 0.2500) (layer "F.Cu") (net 4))
 (segment (start 26.6000 20.6000) (end 26.2000 20.6000) (width 0.2500) (layer "F.Cu") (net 4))
 (segment (start 26.2000 20.6000) (end 26.0000 20.4000) (width 0.2500) (layer "F.Cu") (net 4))
 (segment (start 26.0000 20.4000) (end 26.0000 17.4000) (width 0.2500) (layer "F.Cu") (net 4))
 (segment (start 26.0000 17.4000) (end 23.0000 14.4000) (width 0.2500) (layer "F.Cu") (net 4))
 (segment (start 23.0000 12.4000) (end 23.0000 7.0000) (width 0.2500) (layer "F.Cu") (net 5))
 (segment (start 23.0000 7.0000) (end 22.6000 6.6000) (width 0.2500) (layer "F.Cu") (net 5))
 (segment (start 22.6000 6.6000) (end 22.6000 5.0000) (width 0.2500) (layer "F.Cu") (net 5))
 (via (at 10.4000 19.2000) (size 0.6000) (drill 0.3000) (layers "F.Cu" "B.Cu") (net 1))
 (via (at 17.0000 30.2000) (size 0.6000) (drill 0.3000) (layers "F.Cu" "B.Cu") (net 1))
 (via (at 18.0000 20.4000) (size 0.6000) (drill 0.3000) (layers "F.Cu" "B.Cu") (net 3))
 (via (at 20.0000 18.6000) (size 0.6000) (drill 0.3000) (layers "F.Cu" "B.Cu") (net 3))
 (via (at 9.8000 17.8000) (size 0.6000) (drill 0.3000) (layers "F.Cu" "B.Cu") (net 2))
 (via (at 11.8000 19.6000) (size 0.6000) (drill 0.3000) (layers "F.Cu" "B.Cu") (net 2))
 (via (at 27.4000 16.0000) (size 0.6000) (drill 0.3000) (layers "F.Cu" "B.Cu") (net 2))
 (via (at 27.2000 17.8000) (size 0.6000) (drill 0.3000) (layers "F.Cu" "B.Cu") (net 2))
 (via (at 19.0000 28.2000) (size 0.6000) (drill 0.3000) (layers "F.Cu" "B.Cu") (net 2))
 (via (at 26.6000 24.0000) (size 0.6000) (drill 0.3000) (layers "F.Cu" "B.Cu") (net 6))
 (via (at 25.6000 23.0000) (size 0.6000) (drill 0.3000) (layers "F.Cu" "B.Cu") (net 6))
 (via (at 24.0000 25.2000) (size 0.6000) (drill 0.3000) (layers "F.Cu" "B.Cu") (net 7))
 (via (at 23.0000 24.0000) (size 0.6000) (drill 0.3000) (layers "F.Cu" "B.Cu") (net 7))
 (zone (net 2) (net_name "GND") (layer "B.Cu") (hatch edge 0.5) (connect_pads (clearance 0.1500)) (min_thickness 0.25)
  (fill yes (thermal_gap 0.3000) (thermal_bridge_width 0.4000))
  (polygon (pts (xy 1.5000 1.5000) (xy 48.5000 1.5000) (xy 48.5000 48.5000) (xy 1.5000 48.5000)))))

